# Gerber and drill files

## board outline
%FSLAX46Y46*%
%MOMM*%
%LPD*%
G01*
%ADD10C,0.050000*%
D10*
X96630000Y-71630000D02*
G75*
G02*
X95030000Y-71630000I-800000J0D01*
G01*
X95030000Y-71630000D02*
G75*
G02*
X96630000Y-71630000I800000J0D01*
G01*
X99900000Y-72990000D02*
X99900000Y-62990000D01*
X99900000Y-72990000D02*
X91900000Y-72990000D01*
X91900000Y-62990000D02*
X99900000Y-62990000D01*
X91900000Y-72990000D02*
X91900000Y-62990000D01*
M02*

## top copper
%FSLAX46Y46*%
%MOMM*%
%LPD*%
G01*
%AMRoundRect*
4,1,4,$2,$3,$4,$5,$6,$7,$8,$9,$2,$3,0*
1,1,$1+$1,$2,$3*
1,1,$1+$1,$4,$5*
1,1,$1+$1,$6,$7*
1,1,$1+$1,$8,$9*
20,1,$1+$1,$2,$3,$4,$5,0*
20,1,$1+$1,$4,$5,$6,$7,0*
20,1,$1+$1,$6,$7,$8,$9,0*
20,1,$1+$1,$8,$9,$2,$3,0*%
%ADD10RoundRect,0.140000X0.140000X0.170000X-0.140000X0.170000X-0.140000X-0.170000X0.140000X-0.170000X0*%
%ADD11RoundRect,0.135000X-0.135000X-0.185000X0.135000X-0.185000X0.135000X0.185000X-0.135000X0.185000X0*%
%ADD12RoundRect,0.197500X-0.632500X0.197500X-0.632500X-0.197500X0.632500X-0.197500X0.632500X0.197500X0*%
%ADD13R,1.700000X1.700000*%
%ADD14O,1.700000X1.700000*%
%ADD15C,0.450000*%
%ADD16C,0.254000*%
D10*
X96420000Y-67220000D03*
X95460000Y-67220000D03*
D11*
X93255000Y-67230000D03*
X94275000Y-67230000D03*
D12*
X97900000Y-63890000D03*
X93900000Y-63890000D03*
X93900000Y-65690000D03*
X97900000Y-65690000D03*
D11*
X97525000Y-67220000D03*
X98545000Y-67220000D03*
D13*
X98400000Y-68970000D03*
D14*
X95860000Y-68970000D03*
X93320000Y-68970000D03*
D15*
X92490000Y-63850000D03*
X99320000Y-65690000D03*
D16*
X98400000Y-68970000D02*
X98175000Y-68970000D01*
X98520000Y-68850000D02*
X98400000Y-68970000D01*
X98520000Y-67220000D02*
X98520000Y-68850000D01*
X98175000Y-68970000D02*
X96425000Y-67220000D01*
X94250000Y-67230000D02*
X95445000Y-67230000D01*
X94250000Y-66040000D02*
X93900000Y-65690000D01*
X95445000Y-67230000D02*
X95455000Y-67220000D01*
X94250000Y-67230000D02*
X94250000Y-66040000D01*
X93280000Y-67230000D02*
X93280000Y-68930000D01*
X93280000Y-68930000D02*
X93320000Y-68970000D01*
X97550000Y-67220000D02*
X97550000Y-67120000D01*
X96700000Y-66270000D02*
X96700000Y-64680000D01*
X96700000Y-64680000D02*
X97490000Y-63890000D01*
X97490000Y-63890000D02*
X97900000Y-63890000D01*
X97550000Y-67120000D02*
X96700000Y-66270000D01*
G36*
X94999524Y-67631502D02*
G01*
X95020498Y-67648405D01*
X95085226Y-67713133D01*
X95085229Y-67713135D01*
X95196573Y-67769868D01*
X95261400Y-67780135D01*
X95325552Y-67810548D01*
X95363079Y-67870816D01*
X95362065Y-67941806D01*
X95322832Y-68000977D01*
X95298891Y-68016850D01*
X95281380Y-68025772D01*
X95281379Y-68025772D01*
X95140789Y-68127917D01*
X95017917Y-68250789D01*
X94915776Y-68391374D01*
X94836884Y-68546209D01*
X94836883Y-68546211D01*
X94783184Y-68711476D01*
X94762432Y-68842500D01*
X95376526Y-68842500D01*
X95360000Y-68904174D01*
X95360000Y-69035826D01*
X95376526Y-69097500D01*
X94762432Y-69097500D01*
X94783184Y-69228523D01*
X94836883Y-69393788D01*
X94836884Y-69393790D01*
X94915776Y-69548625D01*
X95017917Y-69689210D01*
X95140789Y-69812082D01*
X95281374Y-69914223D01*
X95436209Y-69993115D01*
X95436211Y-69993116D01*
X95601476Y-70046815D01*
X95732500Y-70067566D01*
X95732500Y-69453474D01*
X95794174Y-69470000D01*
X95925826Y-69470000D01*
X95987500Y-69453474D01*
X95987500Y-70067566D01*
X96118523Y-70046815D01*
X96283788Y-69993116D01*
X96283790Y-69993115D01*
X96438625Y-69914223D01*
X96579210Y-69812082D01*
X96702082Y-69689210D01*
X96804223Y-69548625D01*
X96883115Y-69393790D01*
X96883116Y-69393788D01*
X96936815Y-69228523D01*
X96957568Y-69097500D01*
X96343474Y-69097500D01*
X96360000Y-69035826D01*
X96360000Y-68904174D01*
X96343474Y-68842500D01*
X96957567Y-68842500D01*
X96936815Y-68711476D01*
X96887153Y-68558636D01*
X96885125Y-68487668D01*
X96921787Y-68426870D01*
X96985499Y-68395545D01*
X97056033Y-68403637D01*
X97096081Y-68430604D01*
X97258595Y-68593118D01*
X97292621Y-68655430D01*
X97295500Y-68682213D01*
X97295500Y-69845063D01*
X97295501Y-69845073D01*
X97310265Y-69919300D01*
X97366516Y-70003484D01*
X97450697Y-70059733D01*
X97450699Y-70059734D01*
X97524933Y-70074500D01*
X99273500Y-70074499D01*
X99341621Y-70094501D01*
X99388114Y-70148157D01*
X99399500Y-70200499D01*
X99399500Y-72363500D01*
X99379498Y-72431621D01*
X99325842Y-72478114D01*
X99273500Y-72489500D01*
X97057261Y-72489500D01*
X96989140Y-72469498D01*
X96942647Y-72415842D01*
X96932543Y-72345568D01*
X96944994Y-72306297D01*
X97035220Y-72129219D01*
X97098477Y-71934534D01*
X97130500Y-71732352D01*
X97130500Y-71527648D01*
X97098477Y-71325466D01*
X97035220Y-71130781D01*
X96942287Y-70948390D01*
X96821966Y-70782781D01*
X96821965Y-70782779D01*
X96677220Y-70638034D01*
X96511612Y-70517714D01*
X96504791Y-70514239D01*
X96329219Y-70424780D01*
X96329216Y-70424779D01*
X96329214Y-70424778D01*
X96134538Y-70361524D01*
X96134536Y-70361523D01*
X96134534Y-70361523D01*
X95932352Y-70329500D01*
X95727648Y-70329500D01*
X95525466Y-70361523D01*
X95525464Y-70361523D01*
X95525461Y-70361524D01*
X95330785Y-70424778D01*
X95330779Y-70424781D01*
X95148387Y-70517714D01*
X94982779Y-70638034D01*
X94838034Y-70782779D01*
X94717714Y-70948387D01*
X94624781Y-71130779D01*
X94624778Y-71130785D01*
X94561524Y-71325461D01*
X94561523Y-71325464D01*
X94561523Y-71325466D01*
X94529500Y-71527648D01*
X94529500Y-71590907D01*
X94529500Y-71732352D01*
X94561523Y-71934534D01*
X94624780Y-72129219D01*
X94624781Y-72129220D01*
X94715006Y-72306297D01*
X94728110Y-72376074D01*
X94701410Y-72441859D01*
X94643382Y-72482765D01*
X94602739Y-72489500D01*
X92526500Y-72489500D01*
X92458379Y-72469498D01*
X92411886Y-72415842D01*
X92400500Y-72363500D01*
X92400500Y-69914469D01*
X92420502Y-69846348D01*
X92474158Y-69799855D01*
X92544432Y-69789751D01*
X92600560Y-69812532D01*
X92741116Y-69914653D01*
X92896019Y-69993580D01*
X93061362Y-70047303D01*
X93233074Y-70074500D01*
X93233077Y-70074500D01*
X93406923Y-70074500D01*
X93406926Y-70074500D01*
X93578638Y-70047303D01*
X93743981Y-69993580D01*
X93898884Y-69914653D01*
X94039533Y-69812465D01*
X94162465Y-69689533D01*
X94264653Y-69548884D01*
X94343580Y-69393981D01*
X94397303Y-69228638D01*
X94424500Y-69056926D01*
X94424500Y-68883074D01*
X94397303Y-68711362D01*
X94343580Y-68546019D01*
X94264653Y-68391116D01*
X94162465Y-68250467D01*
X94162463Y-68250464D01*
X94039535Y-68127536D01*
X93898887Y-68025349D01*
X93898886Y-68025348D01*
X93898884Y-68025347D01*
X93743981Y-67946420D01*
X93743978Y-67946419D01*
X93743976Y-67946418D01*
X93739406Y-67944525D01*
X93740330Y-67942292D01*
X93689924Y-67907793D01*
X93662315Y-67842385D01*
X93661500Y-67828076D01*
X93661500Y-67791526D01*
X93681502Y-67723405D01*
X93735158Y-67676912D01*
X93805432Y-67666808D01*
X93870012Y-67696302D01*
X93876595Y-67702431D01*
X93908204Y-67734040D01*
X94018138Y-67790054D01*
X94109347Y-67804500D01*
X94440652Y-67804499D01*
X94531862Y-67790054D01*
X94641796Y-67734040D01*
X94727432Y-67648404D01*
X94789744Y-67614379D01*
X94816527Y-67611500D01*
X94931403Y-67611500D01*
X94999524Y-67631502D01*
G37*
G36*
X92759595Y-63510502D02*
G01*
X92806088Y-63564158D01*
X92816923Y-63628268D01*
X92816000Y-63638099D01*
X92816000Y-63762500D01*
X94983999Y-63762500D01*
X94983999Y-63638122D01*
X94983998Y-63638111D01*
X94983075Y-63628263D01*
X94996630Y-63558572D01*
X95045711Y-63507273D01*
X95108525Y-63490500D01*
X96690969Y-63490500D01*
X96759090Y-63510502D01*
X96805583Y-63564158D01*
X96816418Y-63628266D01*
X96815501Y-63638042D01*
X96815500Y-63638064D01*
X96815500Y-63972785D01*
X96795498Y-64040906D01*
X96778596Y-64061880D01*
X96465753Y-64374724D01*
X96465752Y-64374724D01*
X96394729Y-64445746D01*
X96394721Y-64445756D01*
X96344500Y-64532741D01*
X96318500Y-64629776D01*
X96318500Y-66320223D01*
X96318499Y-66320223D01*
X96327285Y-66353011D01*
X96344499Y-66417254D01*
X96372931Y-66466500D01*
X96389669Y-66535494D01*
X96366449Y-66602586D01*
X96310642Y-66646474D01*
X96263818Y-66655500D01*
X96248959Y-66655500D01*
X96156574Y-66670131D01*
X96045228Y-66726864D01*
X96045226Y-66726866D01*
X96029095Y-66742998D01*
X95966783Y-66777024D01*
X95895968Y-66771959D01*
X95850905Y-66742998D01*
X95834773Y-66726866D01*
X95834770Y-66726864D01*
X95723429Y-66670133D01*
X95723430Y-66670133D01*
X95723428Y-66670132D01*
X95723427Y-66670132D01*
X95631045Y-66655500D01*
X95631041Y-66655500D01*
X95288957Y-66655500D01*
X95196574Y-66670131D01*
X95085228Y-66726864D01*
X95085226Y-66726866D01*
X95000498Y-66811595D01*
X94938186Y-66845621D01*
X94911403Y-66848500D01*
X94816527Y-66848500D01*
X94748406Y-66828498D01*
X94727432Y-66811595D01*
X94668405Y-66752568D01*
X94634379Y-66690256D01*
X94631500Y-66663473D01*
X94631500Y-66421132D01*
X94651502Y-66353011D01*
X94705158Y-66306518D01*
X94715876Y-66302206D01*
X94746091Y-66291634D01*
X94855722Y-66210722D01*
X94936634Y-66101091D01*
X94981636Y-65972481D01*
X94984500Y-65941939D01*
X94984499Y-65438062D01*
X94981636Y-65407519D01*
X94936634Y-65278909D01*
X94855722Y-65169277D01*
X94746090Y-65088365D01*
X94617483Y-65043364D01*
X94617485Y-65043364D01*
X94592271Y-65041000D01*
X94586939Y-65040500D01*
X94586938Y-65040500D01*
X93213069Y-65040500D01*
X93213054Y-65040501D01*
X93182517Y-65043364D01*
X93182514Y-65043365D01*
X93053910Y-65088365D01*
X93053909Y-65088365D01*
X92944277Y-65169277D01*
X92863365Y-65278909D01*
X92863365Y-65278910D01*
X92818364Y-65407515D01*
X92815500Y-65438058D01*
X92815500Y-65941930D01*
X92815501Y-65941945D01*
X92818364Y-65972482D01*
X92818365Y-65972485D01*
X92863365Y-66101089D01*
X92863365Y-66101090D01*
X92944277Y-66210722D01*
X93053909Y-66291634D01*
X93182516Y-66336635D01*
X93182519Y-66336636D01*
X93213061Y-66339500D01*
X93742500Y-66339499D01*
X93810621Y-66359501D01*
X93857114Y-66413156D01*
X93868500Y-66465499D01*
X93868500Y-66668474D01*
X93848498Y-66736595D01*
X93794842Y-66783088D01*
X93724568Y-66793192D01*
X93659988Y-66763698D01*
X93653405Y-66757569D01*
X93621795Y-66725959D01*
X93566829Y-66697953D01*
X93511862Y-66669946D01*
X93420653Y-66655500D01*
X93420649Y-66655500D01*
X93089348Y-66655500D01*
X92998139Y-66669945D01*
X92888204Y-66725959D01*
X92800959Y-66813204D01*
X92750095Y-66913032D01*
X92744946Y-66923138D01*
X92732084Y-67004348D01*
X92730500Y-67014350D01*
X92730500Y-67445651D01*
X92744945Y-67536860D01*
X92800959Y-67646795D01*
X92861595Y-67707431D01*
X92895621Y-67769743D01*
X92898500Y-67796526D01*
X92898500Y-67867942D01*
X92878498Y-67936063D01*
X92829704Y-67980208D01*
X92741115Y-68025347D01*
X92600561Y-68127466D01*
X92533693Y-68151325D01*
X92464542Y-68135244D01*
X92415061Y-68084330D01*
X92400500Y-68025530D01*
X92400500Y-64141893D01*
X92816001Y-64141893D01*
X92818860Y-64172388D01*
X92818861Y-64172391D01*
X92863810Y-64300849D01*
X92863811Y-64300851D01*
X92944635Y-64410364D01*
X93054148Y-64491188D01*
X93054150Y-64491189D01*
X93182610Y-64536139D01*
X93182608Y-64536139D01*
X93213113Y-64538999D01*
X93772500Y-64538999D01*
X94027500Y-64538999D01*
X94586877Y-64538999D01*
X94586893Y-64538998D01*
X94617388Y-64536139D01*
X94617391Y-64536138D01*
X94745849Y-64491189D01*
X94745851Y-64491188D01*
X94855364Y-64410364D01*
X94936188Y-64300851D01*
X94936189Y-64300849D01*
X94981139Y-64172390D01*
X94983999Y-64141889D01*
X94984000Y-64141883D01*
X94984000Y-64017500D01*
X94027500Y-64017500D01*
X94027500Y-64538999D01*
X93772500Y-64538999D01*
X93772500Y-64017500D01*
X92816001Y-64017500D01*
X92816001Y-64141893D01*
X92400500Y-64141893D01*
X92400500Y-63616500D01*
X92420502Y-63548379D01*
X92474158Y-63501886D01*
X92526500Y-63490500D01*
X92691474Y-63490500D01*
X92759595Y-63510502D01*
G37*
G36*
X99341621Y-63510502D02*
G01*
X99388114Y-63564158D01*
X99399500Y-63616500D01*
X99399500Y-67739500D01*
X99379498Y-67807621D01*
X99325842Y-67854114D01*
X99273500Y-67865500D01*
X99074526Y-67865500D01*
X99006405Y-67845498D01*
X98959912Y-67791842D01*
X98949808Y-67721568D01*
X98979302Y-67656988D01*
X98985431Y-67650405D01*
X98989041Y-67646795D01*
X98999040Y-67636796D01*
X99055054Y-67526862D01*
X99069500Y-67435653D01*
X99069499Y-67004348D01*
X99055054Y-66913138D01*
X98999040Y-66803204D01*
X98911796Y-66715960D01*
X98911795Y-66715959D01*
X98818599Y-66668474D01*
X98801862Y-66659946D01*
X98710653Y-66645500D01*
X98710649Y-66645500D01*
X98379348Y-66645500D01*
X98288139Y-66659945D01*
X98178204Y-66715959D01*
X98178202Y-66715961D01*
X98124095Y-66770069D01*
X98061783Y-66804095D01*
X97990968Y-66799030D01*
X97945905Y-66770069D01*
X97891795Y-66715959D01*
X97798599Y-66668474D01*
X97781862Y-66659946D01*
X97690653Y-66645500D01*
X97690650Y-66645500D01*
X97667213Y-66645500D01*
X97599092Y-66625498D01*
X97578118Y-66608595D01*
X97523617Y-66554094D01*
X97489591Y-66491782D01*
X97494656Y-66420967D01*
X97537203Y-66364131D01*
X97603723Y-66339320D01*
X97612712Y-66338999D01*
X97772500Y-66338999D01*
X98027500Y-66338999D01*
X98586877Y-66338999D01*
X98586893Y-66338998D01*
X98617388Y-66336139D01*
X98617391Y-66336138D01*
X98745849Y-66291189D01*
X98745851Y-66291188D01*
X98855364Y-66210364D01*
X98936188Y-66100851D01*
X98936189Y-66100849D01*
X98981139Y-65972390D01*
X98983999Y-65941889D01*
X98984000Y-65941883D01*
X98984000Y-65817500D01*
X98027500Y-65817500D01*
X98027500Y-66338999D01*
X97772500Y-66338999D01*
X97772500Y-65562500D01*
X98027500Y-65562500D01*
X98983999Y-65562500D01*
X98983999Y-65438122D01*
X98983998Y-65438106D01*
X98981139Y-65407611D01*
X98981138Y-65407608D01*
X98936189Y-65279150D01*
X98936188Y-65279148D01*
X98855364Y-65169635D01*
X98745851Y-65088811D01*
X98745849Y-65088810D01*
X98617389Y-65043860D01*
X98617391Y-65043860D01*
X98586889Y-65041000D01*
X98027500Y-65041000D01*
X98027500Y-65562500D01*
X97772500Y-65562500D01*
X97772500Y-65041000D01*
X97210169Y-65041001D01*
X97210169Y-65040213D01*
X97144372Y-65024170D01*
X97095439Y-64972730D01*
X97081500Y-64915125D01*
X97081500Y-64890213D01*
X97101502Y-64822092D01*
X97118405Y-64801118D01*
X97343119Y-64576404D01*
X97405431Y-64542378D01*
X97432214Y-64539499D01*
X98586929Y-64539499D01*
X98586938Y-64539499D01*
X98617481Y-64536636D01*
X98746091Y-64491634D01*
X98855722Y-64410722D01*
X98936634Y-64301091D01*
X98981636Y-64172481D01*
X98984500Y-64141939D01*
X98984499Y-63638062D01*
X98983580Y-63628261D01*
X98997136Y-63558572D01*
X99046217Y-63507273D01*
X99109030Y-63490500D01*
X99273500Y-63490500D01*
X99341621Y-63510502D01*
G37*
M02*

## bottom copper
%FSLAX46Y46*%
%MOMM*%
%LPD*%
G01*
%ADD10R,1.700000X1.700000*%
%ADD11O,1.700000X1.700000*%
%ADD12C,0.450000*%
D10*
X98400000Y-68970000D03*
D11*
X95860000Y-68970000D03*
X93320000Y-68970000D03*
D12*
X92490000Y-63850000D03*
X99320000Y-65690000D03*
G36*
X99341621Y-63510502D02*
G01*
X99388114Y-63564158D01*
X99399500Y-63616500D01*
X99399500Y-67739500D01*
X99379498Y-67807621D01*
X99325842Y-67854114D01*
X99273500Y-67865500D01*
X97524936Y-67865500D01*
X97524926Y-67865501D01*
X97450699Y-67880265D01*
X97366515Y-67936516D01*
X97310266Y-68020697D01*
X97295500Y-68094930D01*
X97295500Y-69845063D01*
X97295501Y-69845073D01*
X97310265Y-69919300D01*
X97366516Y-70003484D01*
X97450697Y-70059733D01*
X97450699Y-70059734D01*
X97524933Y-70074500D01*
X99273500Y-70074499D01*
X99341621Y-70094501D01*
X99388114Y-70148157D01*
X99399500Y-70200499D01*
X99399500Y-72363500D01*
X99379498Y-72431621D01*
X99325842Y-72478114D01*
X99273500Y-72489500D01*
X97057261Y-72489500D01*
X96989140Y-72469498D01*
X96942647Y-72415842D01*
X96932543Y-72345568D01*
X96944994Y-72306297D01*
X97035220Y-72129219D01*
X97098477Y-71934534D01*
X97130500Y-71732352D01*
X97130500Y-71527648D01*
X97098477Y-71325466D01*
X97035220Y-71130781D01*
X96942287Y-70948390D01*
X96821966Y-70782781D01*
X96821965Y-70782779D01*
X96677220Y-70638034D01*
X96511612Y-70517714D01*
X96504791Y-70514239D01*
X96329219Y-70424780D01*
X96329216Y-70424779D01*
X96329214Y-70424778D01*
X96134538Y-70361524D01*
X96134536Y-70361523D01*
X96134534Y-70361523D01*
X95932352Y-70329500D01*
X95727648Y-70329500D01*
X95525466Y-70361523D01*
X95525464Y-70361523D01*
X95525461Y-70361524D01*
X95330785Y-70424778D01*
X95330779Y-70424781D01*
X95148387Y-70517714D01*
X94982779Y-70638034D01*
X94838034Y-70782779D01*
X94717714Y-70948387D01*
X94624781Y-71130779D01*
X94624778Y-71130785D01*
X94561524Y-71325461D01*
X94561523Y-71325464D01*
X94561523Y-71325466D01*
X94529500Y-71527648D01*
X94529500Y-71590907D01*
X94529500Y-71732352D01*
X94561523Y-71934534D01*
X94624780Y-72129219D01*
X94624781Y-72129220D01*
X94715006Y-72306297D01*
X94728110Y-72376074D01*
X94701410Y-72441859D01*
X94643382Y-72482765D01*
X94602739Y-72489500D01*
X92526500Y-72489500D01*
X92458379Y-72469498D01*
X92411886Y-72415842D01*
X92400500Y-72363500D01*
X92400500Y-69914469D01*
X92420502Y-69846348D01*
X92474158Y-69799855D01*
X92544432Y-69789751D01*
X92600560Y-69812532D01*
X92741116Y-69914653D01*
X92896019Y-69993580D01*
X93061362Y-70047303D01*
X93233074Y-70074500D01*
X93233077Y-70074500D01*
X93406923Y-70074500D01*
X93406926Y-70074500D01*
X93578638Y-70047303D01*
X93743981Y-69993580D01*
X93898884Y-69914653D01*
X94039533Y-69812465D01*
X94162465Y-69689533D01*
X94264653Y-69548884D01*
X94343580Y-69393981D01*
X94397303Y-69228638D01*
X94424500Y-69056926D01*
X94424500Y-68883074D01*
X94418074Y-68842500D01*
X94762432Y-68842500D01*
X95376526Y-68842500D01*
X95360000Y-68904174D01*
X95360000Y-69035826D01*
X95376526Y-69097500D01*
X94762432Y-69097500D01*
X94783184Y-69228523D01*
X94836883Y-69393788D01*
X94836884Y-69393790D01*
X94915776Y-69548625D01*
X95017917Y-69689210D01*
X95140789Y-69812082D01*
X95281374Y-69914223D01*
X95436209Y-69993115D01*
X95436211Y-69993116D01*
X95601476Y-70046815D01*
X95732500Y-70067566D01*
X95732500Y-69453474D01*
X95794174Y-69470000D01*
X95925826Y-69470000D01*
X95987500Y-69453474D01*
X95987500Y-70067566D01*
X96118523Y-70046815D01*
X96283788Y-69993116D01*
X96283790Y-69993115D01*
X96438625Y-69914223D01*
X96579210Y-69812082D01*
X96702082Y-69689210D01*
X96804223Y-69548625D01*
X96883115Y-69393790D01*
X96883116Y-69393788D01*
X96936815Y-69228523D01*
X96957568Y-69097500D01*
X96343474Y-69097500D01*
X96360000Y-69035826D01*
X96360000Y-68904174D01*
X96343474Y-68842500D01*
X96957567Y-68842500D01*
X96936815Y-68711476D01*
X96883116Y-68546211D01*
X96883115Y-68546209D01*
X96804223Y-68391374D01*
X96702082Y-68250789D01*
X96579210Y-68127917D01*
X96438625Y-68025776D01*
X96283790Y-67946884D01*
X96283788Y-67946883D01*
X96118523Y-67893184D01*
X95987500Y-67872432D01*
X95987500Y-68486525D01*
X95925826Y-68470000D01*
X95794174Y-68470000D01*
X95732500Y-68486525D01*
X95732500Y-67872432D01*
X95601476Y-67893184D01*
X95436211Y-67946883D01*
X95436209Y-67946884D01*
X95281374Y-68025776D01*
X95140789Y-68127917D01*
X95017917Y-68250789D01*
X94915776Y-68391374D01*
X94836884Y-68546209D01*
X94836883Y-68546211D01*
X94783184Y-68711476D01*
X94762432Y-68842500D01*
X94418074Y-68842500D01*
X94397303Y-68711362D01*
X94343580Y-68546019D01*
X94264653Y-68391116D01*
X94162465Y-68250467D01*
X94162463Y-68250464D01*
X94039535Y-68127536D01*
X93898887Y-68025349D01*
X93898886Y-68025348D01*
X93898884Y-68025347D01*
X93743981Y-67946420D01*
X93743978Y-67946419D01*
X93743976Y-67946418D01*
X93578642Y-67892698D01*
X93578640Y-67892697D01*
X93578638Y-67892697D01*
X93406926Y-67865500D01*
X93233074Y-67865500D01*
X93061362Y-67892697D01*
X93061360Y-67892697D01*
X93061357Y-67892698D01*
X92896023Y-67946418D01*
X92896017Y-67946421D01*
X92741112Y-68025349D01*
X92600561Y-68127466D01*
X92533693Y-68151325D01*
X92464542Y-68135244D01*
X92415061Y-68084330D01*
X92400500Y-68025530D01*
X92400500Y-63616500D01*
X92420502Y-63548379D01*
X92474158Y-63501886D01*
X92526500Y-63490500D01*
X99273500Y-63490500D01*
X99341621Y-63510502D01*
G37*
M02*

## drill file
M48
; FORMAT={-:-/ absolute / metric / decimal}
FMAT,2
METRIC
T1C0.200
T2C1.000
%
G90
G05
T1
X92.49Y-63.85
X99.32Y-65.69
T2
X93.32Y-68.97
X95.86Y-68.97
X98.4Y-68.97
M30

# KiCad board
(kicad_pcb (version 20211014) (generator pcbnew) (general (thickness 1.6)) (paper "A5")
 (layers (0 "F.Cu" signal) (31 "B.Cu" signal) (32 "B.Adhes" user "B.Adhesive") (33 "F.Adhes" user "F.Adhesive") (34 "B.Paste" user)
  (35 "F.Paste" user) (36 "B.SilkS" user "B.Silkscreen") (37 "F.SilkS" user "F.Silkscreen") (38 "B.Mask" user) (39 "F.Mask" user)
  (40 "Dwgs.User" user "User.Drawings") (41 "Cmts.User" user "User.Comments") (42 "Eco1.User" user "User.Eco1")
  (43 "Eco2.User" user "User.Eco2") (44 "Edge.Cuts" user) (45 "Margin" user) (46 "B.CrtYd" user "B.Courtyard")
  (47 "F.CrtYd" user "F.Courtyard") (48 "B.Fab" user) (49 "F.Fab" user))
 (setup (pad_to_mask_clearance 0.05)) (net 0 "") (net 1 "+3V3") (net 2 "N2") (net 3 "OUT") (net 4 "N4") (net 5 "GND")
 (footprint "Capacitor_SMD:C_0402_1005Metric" (layer "F.Cu") (at 95.94 67.22 180)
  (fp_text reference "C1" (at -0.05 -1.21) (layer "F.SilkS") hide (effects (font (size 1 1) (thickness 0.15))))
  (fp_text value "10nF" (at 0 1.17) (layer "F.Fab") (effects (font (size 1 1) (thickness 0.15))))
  (pad "1" smd roundrect (at -0.48 0 180) (size 0.56 0.62) (layers "F.Cu" "F.Paste" "F.Mask") (roundrect_rratio 0.25) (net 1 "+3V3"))
  (pad "2" smd roundrect (at 0.48 0 180) (size 0.56 0.62) (layers "F.Cu" "F.Paste" "F.Mask") (roundrect_rratio 0.25) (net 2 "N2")))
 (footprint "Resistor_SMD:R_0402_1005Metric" (layer "F.Cu") (at 93.765 67.23)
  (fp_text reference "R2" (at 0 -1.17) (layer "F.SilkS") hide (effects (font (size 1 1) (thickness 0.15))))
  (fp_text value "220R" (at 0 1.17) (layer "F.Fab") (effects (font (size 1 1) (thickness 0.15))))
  (pad "1" smd roundrect (at -0.51 0) (size 0.54 0.64) (layers "F.Cu" "F.Paste" "F.Mask") (roundrect_rratio 0.25) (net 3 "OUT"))
  (pad "2" smd roundrect (at 0.51 0) (size 0.54 0.64) (layers "F.Cu" "F.Paste" "F.Mask") (roundrect_rratio 0.25) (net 2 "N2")))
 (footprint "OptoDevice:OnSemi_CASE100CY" (layer "F.Cu") (at 95.9 64.79 -90)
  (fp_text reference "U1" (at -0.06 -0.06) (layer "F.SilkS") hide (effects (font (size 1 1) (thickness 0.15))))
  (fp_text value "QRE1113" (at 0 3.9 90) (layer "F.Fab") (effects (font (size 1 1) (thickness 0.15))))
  (pad "1" smd roundrect (at -0.9 -2 270) (size 0.79 1.66) (layers "F.Cu" "F.Paste" "F.Mask") (roundrect_rratio 0.25) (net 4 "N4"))
  (pad "2" smd roundrect (at -0.9 2 270) (size 0.79 1.66) (layers "F.Cu" "F.Paste" "F.Mask") (roundrect_rratio 0.25) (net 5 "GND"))
  (pad "3" smd roundrect (at 0.9 2 270) (size 0.79 1.66) (layers "F.Cu" "F.Paste" "F.Mask") (roundrect_rratio 0.25) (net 2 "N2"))
  (pad "4" smd roundrect (at 0.9 -2 270) (size 0.79 1.66) (layers "F.Cu" "F.Paste" "F.Mask") (roundrect_rratio 0.25) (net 5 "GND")))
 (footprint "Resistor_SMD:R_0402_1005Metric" (layer "F.Cu") (at 98.035 67.22)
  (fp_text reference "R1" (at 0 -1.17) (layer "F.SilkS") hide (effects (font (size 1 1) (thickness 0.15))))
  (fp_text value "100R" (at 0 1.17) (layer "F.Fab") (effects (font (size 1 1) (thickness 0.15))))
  (pad "1" smd roundrect (at -0.51 0) (size 0.54 0.64) (layers "F.Cu" "F.Paste" "F.Mask") (roundrect_rratio 0.25) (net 4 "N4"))
  (pad "2" smd roundrect (at 0.51 0) (size 0.54 0.64) (layers "F.Cu" "F.Paste" "F.Mask") (roundrect_rratio 0.25) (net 1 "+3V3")))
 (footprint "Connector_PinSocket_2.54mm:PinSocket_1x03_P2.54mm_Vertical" (layer "B.Cu") (at 98.4 68.97 90)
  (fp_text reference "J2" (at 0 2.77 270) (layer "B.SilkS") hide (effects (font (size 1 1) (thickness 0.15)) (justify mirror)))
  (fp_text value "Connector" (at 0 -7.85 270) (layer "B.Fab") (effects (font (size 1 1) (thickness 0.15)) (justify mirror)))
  (pad "1" thru_hole rect locked (at 0 0 90) (size 1.7 1.7) (drill 1) (layers *.Cu *.Mask) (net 1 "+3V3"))
  (pad "2" thru_hole oval locked (at 0 -2.54 90) (size 1.7 1.7) (drill 1) (layers *.Cu *.Mask) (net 5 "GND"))
  (pad "3" thru_hole oval locked (at 0 -5.08 90) (size 1.7 1.7) (drill 1) (layers *.Cu *.Mask) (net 3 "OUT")))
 (gr_circle (center 95.83 71.63) (end 96.63 71.63) (layer "Edge.Cuts") (width 0.05) (fill none))
 (gr_line (start 99.9 72.99) (end 99.9 62.99) (layer "Edge.Cuts") (width 0.05))
 (gr_line (start 99.9 72.99) (end 91.9 72.99) (layer "Edge.Cuts") (width 0.05))
 (gr_line (start 91.9 62.99) (end 99.9 62.99) (layer "Edge.Cuts") (width 0.05))
 (gr_line (start 91.9 72.99) (end 91.9 62.99) (layer "Edge.Cuts") (width 0.05))
 (segment (start 98.4 68.97) (end 98.175 68.97) (width 0.254) (layer "F.Cu") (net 1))
 (segment (start 98.52 68.85) (end 98.4 68.97) (width 0.254) (layer "F.Cu") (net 1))
 (segment (start 98.52 67.22) (end 98.52 68.85) (width 0.254) (layer "F.Cu") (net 1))
 (segment (start 98.175 68.97) (end 96.425 67.22) (width 0.254) (layer "F.Cu") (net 1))
 (via (at 92.49 63.85) (size 0.45) (drill 0.2) (layers "F.Cu" "B.Cu") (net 5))
 (via (at 99.32 65.69) (size 0.45) (drill 0.2) (layers "F.Cu" "B.Cu") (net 5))
 (segment (start 94.25 67.23) (end 95.445 67.23) (width 0.254) (layer "F.Cu") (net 2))
 (segment (start 94.25 66.04) (end 93.9 65.69) (width 0.254) (layer "F.Cu") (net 2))
 (segment (start 95.445 67.23) (end 95.455 67.22) (width 0.254) (layer "F.Cu") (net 2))
 (segment (start 94.25 67.23) (end 94.25 66.04) (width 0.254) (layer "F.Cu") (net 2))
 (segment (start 93.28 67.23) (end 93.28 68.93) (width 0.254) (layer "F.Cu") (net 3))
 (segment (start 93.28 68.93) (end 93.32 68.97) (width 0.254) (layer "F.Cu") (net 3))
 (segment (start 97.55 67.22) (end 97.55 67.12) (width 0.254) (layer "F.Cu") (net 4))
 (segment (start 96.7 66.27) (end 96.7 64.68) (width 0.254) (layer "F.Cu") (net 4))
 (segment (start 96.7 64.68) (end 97.49 63.89) (width 0.254) (layer "F.Cu") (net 4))
 (segment (start 97.49 63.89) (end 97.9 63.89) (width 0.254) (layer "F.Cu") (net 4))
 (segment (start 97.55 67.12) (end 96.7 66.27) (width 0.254) (layer "F.Cu") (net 4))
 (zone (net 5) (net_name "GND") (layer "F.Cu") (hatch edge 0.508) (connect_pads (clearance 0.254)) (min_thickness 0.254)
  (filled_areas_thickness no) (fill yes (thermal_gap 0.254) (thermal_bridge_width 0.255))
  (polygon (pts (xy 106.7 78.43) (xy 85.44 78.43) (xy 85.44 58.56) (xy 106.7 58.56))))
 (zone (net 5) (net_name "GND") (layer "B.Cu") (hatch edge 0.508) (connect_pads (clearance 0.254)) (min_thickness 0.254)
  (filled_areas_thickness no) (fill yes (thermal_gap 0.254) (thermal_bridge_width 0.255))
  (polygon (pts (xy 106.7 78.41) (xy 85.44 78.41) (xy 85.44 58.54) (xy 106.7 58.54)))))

